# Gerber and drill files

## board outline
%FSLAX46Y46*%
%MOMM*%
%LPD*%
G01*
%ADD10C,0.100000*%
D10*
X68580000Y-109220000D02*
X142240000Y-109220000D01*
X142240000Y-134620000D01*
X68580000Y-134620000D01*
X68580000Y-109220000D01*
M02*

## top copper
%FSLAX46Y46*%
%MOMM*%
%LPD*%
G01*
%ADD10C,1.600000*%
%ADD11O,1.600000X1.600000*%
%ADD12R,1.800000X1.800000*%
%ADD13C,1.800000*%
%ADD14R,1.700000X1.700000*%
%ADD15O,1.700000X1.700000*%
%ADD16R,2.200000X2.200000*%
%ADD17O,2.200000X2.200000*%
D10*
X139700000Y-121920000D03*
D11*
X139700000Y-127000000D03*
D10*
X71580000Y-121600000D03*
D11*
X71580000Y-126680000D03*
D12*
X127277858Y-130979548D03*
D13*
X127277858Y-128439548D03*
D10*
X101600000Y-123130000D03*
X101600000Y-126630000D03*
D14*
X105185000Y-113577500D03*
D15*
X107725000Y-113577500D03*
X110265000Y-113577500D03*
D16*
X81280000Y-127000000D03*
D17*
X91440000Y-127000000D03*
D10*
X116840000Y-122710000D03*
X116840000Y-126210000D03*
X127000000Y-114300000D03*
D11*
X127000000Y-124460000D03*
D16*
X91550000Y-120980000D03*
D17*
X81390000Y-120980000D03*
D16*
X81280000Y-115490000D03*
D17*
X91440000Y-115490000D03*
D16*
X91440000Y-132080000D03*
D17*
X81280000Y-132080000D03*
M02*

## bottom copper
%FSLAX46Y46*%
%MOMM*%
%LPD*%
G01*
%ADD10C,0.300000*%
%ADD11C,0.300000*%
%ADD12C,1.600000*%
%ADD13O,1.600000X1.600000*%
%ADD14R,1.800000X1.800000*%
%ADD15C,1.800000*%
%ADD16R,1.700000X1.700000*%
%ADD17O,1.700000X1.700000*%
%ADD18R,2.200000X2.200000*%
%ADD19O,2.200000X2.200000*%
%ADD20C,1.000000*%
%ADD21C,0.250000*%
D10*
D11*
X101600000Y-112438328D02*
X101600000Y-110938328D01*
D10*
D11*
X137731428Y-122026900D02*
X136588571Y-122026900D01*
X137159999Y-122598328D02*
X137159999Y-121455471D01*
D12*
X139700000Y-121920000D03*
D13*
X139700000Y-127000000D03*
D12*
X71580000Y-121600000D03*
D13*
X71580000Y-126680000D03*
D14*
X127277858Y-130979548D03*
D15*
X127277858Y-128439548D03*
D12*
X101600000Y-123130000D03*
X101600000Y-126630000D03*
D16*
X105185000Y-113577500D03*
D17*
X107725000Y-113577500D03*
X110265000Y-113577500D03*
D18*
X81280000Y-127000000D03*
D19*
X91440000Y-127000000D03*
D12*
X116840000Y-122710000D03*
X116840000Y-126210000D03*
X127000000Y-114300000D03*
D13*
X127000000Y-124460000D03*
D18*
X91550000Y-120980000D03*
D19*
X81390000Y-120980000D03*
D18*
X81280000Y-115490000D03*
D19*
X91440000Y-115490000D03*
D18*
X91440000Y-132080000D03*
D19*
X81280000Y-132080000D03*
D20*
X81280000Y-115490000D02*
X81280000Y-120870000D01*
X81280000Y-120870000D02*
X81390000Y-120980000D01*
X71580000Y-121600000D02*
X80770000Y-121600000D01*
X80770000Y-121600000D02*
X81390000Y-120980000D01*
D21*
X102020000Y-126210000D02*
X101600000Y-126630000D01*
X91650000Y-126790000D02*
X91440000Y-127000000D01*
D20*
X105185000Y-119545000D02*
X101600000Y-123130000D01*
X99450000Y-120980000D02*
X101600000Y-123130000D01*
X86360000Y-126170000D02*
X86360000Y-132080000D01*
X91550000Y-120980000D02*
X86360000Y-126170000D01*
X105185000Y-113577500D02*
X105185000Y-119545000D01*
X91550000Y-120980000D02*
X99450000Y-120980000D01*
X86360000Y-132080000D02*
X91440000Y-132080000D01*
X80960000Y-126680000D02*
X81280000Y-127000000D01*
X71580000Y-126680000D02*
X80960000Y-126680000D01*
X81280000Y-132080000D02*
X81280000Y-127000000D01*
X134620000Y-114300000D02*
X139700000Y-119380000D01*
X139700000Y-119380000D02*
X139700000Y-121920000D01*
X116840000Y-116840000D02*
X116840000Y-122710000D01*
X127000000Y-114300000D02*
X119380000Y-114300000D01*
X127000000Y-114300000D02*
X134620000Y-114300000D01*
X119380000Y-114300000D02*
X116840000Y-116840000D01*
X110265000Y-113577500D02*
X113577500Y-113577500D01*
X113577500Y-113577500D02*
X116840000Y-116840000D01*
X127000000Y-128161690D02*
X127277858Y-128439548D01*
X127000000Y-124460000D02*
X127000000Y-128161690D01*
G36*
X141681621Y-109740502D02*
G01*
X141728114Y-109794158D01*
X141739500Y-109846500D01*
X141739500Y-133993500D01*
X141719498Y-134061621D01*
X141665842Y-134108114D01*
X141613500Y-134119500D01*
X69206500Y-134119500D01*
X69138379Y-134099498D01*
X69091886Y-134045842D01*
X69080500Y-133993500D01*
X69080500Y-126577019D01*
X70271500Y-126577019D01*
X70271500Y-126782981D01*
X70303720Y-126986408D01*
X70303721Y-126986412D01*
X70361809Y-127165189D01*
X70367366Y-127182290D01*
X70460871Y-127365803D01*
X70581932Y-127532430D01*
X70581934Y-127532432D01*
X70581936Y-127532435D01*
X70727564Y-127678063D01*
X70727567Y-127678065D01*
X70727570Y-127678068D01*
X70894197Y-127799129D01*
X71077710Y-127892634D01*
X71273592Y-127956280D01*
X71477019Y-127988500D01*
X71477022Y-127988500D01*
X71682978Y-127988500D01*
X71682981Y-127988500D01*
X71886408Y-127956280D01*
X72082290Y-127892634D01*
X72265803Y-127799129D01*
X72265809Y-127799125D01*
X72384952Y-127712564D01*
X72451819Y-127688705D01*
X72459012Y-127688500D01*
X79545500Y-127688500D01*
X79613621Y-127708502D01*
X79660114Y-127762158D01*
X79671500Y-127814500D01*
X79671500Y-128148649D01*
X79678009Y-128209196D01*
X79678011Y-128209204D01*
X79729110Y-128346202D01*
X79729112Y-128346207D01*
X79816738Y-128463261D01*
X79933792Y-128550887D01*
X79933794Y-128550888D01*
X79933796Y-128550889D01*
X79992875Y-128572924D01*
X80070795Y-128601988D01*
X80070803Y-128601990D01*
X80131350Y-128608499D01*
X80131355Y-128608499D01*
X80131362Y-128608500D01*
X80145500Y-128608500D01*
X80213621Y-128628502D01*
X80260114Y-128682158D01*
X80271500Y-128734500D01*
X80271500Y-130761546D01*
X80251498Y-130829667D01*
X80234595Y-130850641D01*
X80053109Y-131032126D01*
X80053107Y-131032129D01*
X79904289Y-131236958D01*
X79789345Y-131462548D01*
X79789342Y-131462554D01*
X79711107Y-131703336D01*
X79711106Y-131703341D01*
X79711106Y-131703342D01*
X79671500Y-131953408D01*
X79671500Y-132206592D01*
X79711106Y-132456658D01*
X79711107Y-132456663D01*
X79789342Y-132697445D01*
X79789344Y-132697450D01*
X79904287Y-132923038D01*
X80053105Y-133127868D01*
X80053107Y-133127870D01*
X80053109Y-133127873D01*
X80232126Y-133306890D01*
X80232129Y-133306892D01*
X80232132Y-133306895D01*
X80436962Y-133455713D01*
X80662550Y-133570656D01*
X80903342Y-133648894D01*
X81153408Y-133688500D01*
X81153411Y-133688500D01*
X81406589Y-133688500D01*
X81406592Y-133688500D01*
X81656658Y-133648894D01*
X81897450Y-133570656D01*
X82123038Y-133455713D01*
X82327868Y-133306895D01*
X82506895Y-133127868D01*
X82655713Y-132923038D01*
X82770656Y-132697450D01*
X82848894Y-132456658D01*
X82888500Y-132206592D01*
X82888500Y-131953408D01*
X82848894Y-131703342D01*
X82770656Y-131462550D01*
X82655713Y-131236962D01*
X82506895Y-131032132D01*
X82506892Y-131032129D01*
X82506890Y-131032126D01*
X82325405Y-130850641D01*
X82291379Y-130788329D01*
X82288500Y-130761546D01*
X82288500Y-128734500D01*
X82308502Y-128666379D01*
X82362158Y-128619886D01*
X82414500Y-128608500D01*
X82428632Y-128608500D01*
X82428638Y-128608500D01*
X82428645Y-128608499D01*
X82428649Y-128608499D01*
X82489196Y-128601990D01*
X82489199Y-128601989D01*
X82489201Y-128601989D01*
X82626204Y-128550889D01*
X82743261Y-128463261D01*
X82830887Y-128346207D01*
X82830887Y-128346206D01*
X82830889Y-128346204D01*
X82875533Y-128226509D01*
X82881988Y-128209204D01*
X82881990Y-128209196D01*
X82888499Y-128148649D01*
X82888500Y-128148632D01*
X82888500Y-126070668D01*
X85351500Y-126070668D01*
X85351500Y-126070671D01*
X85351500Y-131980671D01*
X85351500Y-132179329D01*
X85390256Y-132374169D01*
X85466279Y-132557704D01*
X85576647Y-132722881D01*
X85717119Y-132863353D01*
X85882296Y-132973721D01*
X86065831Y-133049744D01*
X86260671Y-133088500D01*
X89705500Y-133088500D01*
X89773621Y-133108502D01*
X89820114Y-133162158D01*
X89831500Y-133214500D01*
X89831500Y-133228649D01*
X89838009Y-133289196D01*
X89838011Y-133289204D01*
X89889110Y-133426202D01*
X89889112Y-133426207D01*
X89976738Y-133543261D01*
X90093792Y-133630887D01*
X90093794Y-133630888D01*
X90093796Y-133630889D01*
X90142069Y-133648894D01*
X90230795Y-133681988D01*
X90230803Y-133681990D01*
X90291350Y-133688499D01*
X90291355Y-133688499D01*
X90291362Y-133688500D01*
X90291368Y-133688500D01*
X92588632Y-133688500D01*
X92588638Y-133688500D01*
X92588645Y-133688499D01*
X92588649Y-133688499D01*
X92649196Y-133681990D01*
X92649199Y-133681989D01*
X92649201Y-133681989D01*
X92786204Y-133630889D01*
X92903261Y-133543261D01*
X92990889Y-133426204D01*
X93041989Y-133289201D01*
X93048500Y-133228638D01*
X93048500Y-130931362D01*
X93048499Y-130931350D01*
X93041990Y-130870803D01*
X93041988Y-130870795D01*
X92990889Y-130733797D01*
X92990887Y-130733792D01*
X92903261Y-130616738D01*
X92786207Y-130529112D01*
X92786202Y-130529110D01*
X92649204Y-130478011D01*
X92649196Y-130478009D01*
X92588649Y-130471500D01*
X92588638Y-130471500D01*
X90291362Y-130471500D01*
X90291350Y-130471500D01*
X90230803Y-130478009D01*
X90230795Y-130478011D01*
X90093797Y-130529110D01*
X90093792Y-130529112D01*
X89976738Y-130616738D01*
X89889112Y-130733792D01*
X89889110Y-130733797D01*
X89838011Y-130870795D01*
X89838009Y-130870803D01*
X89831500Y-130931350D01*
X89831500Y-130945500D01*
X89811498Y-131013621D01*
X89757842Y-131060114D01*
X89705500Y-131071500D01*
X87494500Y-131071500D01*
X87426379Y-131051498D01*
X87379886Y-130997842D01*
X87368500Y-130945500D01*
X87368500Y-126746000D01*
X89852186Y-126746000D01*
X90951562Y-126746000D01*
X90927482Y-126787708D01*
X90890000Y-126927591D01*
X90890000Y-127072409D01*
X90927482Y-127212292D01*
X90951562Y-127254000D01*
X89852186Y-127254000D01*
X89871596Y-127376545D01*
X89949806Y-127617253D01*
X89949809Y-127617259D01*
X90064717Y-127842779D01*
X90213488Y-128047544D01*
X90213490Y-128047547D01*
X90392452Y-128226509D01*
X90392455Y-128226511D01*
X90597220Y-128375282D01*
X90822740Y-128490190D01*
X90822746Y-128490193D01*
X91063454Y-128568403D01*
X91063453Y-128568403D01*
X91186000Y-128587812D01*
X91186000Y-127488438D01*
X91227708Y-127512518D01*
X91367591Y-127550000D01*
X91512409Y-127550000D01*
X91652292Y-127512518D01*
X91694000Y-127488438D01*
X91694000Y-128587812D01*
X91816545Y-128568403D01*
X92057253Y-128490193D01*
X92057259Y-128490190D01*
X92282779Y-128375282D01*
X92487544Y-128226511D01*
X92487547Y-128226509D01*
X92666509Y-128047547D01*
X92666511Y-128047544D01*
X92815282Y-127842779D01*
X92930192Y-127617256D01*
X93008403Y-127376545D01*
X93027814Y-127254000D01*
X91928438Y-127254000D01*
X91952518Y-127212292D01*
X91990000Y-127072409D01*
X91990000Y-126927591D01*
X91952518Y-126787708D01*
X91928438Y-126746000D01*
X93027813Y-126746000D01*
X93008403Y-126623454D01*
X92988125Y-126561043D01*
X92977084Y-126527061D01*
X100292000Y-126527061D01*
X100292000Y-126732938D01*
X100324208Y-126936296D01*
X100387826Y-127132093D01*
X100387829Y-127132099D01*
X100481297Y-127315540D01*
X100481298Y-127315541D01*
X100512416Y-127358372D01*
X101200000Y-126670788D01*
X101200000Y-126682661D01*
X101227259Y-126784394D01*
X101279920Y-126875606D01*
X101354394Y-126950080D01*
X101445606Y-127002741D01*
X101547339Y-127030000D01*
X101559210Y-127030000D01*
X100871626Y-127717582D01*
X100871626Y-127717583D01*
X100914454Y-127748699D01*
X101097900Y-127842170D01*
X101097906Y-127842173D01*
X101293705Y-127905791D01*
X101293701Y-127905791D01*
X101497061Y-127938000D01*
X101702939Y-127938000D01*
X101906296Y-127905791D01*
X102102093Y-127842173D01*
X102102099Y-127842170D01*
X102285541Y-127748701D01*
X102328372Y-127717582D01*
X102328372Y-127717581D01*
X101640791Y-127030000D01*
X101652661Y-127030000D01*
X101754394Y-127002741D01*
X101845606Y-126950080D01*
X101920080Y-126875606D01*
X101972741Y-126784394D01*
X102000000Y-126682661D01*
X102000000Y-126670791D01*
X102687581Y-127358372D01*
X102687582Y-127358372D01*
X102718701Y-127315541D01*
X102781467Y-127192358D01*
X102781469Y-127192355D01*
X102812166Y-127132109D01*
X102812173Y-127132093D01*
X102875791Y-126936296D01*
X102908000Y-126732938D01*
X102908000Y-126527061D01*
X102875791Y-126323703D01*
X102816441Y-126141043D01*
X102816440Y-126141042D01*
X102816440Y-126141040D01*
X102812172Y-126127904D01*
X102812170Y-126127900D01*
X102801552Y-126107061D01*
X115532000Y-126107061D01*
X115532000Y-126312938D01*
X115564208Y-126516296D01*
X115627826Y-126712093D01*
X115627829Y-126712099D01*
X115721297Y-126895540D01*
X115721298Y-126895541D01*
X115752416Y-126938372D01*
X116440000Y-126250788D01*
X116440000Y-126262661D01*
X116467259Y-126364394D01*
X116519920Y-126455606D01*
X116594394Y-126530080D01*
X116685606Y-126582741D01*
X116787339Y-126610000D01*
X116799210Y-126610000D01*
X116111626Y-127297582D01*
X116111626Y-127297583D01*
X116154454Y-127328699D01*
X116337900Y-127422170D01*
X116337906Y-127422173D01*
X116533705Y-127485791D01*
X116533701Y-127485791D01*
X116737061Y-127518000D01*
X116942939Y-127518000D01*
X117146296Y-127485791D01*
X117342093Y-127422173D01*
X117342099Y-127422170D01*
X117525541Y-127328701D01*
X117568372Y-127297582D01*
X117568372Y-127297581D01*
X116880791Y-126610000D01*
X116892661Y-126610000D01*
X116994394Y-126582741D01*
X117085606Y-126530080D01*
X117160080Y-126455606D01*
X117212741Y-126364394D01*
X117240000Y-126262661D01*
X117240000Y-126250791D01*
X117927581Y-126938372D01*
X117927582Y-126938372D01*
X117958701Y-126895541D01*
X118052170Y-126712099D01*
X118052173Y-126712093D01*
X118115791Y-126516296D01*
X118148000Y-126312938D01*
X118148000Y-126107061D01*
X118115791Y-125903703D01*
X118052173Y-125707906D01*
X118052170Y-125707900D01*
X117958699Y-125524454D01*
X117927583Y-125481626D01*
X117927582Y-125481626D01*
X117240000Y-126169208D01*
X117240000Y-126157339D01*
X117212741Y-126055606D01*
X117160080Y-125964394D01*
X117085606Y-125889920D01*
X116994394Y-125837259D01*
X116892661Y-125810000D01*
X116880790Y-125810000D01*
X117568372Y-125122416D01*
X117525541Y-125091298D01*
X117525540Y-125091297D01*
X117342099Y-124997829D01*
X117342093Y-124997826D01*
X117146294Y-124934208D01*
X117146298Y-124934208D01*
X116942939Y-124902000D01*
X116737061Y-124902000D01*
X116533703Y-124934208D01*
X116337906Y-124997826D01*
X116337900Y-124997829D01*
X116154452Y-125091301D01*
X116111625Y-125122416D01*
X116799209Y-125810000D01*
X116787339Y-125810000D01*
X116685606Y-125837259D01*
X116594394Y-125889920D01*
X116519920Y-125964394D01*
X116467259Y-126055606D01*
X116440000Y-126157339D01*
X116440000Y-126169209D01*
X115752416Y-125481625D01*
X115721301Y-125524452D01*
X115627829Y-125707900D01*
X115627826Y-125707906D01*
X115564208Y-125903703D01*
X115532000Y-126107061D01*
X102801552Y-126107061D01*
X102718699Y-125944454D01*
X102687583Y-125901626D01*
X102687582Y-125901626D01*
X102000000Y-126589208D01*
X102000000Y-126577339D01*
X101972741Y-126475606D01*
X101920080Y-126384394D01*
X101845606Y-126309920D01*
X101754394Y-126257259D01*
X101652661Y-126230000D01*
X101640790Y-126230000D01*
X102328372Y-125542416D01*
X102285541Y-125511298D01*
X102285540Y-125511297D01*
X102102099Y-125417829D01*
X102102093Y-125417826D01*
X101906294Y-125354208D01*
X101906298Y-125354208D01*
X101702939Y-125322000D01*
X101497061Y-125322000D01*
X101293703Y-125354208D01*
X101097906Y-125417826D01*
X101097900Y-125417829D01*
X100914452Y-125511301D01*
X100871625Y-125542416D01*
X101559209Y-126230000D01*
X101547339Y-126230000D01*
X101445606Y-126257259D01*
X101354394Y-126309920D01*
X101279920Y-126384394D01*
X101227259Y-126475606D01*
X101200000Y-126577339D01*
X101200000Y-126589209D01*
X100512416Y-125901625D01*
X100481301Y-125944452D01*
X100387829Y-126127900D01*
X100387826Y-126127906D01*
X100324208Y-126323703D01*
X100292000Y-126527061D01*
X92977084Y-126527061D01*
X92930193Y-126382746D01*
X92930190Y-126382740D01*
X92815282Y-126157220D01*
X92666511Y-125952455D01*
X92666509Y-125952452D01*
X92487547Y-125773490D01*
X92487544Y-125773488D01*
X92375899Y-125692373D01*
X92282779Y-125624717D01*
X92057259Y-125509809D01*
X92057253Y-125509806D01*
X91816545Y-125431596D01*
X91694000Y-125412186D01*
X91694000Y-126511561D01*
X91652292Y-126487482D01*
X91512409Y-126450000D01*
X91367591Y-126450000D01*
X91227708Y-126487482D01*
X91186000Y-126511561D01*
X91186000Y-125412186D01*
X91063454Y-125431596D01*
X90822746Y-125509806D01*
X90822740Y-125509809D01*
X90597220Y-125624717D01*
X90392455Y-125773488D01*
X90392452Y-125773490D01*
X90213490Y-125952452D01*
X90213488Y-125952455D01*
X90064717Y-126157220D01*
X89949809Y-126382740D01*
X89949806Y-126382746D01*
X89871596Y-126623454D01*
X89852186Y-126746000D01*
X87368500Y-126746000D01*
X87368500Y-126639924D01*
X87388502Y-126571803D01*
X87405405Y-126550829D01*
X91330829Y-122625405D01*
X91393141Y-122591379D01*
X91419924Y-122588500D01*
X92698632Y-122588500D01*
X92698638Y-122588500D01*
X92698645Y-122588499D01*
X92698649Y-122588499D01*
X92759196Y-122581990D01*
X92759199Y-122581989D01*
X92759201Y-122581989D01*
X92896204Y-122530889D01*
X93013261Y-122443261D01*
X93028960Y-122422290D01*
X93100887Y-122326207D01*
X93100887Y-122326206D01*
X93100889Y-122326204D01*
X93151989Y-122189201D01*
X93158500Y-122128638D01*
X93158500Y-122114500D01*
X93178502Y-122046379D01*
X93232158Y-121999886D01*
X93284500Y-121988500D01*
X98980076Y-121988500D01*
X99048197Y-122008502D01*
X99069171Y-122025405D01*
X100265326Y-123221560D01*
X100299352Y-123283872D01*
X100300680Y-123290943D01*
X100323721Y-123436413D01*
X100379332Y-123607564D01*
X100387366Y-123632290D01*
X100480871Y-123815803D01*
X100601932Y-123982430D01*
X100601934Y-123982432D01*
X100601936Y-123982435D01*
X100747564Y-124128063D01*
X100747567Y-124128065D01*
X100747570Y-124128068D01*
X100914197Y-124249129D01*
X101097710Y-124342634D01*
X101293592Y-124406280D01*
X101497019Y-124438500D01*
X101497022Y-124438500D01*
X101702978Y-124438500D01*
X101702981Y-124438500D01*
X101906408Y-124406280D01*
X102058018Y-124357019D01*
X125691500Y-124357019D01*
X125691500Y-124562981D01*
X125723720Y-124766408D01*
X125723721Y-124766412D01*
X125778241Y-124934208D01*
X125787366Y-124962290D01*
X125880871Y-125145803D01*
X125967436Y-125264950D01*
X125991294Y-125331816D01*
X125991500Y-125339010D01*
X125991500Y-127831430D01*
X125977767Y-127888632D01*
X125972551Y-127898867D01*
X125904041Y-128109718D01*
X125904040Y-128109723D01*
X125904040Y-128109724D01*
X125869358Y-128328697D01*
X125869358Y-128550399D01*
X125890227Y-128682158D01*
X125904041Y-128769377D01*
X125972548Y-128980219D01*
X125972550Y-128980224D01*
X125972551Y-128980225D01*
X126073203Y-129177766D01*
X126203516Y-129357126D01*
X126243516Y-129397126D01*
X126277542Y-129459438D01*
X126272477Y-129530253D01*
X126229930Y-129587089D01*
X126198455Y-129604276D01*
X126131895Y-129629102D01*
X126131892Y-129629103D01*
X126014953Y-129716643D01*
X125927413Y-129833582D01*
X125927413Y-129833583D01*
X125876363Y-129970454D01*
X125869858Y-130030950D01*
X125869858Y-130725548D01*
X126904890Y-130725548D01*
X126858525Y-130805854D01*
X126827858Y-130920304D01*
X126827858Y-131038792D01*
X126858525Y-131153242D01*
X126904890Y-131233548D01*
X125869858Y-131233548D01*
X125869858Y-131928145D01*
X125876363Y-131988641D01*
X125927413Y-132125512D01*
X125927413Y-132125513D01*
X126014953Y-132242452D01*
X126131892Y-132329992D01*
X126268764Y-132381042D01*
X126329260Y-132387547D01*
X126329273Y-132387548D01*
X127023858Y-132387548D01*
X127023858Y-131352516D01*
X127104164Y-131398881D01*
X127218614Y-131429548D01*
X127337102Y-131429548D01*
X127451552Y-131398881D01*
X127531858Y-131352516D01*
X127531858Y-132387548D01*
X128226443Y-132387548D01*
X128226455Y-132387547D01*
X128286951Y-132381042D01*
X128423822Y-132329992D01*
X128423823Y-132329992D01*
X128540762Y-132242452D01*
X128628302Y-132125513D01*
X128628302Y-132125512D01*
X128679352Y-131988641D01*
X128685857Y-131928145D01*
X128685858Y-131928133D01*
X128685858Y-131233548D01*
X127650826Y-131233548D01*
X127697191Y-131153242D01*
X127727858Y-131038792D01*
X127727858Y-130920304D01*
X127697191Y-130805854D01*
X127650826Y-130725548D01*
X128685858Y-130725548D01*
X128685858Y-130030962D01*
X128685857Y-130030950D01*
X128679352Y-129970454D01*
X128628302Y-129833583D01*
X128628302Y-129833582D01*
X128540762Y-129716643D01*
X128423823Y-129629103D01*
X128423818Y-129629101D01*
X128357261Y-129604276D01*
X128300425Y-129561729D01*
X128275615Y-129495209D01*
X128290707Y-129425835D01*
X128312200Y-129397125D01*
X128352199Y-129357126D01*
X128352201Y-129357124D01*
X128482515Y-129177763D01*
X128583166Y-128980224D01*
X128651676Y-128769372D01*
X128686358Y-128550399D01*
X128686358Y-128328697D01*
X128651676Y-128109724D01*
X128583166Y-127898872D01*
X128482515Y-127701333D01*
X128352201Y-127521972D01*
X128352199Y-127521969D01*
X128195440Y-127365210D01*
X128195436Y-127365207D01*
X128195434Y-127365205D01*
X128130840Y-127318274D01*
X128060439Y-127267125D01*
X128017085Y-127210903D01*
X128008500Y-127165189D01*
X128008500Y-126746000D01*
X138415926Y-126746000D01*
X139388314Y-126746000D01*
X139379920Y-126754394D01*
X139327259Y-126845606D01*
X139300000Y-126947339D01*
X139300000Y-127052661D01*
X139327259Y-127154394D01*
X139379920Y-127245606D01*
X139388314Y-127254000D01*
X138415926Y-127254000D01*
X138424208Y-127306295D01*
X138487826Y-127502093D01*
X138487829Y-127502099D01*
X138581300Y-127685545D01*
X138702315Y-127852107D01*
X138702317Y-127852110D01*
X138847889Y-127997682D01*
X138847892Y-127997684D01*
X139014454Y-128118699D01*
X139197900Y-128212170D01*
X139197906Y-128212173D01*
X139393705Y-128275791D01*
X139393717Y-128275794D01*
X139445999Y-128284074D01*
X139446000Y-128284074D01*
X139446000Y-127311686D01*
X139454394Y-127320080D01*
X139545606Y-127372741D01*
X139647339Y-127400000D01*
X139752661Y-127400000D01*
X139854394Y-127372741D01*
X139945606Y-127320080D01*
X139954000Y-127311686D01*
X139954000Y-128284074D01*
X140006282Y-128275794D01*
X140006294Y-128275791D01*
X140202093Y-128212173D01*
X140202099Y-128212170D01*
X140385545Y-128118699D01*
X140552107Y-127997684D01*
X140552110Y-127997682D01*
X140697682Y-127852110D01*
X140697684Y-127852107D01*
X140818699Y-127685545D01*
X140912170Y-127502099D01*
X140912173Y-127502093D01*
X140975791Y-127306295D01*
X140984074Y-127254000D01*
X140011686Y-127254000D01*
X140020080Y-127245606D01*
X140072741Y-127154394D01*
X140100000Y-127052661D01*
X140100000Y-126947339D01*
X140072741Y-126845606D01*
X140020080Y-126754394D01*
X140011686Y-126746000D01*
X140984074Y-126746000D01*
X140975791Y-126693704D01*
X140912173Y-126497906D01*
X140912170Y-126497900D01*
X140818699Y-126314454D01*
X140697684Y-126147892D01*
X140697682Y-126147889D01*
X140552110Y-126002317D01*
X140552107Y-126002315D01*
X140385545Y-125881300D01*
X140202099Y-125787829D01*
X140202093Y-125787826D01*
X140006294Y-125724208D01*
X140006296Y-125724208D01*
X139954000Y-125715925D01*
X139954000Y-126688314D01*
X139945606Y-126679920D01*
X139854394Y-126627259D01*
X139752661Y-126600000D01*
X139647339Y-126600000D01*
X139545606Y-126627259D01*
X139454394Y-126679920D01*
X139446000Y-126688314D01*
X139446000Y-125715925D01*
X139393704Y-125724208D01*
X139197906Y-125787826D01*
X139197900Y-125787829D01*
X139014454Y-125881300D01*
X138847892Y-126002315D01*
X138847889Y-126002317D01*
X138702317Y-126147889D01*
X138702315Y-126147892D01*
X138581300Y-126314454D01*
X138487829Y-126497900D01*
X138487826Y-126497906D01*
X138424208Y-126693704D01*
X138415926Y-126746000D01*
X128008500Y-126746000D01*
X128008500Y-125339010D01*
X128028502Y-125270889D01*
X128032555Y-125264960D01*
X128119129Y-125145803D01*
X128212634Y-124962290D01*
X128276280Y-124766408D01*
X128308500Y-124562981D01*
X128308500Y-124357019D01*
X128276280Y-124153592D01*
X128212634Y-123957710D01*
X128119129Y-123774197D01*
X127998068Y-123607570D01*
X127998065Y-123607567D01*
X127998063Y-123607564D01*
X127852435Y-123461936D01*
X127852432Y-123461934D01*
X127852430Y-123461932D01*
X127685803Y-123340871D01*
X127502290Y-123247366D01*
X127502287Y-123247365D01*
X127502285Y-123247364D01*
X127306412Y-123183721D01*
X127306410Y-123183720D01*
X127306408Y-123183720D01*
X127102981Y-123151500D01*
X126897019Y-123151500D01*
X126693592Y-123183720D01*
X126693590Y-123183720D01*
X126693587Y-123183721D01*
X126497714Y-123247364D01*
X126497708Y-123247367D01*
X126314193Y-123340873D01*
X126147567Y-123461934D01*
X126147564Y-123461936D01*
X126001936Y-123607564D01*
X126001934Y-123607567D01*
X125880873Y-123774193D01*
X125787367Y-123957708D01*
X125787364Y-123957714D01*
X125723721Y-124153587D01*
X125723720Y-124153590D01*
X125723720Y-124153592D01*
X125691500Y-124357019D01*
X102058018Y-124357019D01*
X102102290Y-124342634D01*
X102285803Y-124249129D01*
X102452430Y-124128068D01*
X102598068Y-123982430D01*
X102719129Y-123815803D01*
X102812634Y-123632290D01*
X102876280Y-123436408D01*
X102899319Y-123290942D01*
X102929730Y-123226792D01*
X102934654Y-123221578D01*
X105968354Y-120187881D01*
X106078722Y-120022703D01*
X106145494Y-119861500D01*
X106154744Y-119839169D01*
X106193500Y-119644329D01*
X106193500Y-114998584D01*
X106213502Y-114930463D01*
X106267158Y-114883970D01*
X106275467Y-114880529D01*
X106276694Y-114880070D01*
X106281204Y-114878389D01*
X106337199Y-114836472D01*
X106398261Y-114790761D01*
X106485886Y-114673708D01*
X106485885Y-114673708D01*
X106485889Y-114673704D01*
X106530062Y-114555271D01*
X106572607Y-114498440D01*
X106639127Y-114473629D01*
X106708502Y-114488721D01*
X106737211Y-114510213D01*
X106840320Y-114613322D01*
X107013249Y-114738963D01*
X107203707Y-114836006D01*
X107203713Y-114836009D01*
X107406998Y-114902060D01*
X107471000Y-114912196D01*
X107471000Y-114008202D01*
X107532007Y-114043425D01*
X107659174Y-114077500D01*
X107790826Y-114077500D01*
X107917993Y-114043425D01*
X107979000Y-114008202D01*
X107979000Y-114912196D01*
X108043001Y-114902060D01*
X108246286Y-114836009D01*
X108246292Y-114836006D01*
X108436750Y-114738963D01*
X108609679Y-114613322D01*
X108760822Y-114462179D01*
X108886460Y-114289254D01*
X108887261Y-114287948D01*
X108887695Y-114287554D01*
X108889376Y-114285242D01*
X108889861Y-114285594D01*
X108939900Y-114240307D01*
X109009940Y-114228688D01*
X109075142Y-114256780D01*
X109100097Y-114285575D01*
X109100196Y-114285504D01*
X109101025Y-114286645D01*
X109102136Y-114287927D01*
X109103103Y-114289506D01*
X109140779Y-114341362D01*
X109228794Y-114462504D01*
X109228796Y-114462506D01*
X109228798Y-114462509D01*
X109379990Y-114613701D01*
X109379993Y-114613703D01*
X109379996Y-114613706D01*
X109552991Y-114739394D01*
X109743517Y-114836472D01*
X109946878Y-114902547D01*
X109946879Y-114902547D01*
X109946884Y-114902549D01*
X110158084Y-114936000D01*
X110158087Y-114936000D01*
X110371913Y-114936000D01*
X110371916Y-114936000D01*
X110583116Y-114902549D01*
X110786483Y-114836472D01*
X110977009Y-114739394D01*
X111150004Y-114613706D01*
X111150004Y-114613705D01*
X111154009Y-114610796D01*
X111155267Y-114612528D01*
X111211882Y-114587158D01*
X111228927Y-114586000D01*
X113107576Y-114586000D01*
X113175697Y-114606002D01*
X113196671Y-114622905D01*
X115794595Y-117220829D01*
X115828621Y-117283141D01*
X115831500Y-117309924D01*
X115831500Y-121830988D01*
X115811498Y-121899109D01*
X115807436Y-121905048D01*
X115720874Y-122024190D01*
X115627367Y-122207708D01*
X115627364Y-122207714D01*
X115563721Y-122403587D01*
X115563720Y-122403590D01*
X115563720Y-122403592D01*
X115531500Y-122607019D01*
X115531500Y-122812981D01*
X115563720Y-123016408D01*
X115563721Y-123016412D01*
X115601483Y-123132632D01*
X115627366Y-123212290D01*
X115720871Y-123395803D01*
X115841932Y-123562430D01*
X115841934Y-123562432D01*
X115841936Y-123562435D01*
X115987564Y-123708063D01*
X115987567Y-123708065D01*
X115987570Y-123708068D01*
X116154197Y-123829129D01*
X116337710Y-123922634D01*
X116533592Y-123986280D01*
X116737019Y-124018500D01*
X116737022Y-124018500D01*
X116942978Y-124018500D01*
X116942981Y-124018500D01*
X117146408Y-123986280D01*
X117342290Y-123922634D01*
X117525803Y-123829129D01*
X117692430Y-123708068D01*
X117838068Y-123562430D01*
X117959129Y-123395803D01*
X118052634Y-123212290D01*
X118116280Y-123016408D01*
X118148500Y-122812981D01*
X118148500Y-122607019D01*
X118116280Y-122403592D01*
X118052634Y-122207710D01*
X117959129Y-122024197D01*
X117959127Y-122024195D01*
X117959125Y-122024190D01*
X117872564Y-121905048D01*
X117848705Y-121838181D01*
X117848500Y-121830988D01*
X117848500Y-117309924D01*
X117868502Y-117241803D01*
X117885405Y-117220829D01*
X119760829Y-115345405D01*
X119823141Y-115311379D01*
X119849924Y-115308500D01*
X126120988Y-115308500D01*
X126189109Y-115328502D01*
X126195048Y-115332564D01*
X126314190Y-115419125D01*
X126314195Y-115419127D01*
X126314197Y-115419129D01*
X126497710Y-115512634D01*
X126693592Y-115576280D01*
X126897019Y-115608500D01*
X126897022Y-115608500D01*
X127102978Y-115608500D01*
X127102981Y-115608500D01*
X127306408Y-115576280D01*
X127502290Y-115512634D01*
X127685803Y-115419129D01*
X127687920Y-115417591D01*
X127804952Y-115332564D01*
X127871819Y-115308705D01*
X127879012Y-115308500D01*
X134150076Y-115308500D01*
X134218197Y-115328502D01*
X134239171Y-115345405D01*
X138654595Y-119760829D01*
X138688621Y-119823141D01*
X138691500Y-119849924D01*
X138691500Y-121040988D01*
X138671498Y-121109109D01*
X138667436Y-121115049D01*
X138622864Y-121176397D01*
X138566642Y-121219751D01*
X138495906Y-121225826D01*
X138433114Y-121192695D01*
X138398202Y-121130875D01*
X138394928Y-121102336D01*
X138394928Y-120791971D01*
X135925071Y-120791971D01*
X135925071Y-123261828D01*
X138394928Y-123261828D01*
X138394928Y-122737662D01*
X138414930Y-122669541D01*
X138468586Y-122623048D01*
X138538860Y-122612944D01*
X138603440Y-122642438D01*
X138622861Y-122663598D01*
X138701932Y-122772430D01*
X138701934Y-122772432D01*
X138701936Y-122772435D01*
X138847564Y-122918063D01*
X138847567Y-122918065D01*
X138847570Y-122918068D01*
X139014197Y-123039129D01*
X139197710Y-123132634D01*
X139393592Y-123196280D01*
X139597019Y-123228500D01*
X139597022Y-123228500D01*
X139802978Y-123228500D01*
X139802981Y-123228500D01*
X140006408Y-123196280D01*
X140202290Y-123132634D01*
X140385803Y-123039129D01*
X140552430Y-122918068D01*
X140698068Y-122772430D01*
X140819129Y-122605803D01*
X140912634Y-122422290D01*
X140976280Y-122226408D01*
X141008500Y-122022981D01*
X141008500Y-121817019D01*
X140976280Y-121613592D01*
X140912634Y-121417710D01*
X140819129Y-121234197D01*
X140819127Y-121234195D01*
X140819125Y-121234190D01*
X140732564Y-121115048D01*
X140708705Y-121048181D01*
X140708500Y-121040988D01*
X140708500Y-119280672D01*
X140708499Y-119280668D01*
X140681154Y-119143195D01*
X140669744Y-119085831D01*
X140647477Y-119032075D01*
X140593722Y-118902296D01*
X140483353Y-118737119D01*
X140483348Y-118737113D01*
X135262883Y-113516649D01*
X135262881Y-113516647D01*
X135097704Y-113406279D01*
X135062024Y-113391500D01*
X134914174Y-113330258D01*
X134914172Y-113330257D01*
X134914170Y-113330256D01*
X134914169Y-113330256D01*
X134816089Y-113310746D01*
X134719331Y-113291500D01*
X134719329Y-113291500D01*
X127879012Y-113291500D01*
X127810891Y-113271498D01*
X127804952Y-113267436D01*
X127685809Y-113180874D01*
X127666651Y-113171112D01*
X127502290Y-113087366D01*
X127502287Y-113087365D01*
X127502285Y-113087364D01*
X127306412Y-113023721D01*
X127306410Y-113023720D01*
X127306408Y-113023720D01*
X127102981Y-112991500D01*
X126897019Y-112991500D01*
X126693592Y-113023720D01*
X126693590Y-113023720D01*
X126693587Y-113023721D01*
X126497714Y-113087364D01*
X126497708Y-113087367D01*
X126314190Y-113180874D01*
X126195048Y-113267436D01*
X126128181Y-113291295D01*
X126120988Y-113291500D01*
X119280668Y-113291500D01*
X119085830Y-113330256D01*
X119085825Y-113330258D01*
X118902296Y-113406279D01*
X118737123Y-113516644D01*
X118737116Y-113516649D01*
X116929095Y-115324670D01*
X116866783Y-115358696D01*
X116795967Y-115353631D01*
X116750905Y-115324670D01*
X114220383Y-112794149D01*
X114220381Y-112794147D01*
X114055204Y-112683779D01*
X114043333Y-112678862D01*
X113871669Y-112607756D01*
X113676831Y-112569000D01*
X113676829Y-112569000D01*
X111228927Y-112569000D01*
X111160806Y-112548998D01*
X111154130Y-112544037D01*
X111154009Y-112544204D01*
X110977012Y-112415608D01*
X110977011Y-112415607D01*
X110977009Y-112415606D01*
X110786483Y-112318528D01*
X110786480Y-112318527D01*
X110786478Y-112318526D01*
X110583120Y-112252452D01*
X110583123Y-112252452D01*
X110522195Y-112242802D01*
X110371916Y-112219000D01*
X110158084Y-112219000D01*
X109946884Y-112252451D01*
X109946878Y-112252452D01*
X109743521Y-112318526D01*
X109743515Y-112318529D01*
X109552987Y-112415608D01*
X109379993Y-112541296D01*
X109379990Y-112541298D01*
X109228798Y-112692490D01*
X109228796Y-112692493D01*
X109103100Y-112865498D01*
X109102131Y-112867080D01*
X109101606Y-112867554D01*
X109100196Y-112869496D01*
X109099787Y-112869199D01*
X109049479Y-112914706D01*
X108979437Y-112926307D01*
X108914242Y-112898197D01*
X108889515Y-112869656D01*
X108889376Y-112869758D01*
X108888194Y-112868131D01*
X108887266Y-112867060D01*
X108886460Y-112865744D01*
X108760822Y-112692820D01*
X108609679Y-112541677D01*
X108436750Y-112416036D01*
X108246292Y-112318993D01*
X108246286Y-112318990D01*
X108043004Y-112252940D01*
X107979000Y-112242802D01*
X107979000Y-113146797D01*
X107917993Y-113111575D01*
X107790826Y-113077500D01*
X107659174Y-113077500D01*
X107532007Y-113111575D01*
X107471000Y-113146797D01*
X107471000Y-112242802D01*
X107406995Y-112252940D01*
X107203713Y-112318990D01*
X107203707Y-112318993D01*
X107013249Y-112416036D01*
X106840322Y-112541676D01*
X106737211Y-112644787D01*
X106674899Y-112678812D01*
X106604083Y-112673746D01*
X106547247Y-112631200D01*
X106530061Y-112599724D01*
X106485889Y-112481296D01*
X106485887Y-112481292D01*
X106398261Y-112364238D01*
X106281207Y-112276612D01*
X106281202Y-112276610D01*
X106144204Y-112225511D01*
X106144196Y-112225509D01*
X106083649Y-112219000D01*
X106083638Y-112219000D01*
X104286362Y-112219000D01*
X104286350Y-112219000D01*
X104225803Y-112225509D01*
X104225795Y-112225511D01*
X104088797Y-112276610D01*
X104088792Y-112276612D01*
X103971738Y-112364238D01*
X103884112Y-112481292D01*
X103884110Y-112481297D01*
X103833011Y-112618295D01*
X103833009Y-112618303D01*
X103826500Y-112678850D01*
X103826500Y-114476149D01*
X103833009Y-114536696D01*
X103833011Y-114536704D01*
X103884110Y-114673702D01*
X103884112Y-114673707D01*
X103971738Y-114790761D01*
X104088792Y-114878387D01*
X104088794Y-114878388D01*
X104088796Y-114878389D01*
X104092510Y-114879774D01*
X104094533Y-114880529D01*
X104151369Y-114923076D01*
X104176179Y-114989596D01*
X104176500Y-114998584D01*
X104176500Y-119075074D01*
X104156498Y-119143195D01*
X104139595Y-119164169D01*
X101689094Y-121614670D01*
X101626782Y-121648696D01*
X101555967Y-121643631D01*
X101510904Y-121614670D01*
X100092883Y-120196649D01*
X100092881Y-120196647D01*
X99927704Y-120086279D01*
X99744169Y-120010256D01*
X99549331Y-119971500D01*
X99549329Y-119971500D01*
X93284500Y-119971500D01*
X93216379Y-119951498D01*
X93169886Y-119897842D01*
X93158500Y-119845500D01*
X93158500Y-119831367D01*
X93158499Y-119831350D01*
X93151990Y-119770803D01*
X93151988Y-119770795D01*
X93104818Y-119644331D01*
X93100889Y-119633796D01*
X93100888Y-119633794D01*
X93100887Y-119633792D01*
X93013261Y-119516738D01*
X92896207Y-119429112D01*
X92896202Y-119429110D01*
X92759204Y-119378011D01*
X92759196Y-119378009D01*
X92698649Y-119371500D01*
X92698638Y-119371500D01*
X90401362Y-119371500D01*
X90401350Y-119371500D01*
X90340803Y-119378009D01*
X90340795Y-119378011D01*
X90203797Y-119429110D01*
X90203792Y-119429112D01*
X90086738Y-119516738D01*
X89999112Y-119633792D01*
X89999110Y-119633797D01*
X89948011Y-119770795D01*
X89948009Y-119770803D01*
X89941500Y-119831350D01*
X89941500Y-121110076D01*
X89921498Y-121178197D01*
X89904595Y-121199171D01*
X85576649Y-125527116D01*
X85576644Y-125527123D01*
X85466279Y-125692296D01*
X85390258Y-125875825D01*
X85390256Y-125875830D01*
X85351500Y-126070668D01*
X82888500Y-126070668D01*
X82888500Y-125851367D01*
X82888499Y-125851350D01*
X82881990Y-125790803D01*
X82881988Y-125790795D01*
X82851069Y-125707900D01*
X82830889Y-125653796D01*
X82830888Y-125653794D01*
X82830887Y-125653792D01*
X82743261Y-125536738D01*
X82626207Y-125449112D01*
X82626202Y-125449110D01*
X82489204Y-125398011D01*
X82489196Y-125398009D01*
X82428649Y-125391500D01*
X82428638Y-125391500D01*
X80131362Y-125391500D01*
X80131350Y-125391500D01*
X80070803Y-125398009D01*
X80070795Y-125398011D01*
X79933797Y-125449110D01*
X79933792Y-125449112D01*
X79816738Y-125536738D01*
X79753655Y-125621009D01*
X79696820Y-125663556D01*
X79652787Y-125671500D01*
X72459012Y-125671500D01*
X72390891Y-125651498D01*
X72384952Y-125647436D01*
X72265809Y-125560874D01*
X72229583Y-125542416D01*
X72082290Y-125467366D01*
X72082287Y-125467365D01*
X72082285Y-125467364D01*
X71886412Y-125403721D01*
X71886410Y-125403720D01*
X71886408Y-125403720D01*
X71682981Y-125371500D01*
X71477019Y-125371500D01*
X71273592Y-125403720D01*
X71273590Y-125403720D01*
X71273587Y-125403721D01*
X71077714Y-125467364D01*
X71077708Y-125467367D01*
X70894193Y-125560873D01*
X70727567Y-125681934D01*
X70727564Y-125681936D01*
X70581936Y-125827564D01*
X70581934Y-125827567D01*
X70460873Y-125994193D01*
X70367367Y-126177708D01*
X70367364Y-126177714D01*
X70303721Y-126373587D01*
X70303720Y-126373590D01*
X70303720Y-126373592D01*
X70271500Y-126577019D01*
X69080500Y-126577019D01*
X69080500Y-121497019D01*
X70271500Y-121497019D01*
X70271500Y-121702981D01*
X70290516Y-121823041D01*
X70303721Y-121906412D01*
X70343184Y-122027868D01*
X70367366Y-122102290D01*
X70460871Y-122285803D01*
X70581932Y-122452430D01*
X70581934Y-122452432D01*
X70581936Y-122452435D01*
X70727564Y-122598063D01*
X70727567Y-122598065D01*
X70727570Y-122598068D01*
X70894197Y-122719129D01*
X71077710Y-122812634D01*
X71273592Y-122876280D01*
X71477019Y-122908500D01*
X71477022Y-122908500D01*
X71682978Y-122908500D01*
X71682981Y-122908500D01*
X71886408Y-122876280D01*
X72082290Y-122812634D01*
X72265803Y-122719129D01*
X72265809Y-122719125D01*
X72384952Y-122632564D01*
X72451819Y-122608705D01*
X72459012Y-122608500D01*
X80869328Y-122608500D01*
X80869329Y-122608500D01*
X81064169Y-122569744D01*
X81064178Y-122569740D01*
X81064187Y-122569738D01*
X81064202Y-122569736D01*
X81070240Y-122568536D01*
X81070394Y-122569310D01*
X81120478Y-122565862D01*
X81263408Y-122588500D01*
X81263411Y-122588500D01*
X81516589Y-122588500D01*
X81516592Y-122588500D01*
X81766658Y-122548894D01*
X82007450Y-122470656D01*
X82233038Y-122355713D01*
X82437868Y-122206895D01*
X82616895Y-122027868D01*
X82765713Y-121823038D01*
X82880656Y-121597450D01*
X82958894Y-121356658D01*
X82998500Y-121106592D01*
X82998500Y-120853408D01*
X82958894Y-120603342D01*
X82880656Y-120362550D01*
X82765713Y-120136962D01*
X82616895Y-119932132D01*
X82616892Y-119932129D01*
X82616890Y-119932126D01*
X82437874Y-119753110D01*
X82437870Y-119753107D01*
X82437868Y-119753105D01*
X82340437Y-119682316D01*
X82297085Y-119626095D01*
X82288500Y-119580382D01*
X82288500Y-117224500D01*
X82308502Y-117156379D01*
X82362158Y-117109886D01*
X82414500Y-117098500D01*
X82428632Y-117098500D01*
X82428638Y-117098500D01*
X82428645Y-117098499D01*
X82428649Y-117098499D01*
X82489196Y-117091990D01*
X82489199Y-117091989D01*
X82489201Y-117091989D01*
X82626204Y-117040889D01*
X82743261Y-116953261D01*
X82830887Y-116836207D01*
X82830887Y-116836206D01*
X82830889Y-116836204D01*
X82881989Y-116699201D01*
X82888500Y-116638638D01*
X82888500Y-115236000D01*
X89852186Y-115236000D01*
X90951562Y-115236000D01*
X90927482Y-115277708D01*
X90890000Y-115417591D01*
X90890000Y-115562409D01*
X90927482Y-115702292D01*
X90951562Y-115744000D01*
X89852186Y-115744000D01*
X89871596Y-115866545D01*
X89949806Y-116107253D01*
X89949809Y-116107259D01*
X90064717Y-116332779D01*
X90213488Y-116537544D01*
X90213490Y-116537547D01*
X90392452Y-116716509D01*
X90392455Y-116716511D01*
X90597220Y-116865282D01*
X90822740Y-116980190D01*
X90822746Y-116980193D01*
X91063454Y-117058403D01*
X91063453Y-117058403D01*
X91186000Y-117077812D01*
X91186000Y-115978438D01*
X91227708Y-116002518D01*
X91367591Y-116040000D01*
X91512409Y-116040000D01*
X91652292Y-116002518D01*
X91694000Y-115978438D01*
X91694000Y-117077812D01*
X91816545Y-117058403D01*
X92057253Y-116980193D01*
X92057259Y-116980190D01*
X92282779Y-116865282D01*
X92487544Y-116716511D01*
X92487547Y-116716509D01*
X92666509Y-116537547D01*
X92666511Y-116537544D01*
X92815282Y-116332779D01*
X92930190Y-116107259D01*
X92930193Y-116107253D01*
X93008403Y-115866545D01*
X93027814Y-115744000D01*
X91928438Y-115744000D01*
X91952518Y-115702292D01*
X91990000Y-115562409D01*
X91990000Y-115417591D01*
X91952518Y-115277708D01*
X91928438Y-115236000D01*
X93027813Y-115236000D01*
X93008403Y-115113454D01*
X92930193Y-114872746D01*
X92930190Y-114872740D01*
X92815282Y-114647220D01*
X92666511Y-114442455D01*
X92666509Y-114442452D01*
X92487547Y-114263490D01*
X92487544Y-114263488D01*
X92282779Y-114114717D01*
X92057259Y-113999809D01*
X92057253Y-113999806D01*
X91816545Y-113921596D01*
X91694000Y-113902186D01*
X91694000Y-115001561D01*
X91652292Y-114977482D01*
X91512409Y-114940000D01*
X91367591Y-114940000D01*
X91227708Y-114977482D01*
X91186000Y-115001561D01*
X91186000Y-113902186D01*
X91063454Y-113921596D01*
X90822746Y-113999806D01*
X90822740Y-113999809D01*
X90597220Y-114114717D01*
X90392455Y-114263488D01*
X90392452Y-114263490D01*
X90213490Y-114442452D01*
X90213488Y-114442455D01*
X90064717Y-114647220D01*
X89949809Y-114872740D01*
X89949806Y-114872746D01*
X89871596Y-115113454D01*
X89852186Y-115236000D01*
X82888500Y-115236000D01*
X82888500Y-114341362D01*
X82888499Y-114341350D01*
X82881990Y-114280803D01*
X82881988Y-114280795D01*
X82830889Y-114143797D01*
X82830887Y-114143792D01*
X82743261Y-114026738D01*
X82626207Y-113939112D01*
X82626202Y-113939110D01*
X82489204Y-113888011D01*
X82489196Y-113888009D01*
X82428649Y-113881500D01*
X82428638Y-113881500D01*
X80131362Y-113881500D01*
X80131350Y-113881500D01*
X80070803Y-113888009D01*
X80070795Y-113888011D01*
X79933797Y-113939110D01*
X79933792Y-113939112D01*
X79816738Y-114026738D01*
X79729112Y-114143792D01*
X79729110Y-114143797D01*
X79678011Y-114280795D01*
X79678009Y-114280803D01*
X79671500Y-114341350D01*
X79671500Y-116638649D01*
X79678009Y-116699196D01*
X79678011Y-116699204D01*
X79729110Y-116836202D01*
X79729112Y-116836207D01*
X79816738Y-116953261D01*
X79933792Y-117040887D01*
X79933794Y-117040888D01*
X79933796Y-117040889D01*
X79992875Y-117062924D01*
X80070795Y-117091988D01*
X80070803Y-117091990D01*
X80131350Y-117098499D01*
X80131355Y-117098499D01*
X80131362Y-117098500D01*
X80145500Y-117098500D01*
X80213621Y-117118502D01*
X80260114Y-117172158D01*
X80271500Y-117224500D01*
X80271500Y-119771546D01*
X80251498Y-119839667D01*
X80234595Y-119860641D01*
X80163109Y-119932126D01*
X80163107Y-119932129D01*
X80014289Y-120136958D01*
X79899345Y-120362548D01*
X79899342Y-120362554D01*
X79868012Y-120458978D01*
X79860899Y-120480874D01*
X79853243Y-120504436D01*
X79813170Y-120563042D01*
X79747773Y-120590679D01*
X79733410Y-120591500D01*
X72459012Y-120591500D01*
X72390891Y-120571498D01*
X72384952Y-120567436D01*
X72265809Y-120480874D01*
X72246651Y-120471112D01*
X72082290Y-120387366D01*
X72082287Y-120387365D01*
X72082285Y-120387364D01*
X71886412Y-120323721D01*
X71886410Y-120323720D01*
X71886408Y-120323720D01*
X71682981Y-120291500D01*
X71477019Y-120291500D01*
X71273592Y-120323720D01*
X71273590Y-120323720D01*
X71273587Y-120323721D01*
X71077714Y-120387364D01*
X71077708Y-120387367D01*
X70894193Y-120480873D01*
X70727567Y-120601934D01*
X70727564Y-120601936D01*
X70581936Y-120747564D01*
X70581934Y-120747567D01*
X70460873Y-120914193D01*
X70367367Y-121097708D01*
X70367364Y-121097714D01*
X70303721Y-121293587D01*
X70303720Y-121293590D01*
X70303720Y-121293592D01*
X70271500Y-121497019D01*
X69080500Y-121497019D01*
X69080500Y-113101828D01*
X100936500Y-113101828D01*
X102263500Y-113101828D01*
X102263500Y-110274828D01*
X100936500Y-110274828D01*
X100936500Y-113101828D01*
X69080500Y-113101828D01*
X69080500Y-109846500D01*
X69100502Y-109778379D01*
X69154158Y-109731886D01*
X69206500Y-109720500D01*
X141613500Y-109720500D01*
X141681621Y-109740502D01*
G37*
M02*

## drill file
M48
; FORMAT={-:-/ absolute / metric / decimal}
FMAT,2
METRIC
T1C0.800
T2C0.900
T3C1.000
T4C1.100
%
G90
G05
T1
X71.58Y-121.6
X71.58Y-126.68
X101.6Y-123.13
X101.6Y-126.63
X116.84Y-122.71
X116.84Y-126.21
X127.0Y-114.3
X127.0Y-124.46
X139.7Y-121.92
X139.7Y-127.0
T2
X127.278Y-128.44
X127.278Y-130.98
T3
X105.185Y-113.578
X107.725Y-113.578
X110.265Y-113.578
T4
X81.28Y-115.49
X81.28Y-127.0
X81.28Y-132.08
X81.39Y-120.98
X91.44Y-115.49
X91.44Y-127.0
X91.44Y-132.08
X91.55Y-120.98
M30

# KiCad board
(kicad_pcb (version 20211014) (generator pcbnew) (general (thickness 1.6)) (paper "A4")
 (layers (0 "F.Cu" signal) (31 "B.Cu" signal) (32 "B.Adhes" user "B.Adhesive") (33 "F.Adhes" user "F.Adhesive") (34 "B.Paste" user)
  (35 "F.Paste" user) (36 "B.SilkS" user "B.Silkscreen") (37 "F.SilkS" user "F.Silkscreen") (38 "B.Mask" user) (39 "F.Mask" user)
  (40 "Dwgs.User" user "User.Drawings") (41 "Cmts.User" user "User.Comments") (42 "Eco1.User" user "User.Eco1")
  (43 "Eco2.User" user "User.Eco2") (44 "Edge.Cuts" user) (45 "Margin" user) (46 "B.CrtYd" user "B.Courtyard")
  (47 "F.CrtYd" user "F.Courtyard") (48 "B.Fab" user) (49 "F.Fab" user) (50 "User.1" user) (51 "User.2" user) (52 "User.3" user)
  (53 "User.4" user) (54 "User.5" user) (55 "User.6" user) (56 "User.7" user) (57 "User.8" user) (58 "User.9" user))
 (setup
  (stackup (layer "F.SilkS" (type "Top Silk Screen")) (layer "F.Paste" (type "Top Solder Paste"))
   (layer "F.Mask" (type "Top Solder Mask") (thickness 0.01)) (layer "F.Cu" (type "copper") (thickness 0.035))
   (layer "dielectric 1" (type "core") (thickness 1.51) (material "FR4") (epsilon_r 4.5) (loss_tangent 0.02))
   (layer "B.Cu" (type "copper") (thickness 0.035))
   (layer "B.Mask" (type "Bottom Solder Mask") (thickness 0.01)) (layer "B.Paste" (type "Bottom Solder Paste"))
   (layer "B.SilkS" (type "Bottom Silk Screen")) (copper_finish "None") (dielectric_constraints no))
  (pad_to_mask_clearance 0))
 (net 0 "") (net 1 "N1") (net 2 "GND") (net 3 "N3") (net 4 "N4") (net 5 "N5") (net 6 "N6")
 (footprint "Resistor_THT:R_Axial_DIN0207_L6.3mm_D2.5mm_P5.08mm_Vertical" (layer "F.Cu") (at 139.7 121.92 -90)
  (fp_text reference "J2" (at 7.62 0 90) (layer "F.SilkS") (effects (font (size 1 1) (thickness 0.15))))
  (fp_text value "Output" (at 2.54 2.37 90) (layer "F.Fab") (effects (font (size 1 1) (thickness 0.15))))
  (pad "1" thru_hole circle (at 0 0 270) (size 1.6 1.6) (drill 0.8) (layers *.Cu *.Mask) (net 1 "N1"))
  (pad "2" thru_hole oval (at 5.08 0 270) (size 1.6 1.6) (drill 0.8) (layers *.Cu *.Mask) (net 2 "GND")))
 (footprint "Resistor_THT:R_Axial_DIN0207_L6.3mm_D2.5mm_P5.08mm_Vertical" (layer "F.Cu") (at 71.58 121.6 -90)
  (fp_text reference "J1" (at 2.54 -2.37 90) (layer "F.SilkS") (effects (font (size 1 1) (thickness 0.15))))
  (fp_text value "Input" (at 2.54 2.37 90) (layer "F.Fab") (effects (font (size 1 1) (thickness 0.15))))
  (pad "1" thru_hole circle (at 0 0 270) (size 1.6 1.6) (drill 0.8) (layers *.Cu *.Mask) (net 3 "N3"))
  (pad "2" thru_hole oval (at 5.08 0 270) (size 1.6 1.6) (drill 0.8) (layers *.Cu *.Mask) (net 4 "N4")))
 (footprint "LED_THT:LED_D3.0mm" (layer "F.Cu") (at 127.277858 130.979548 90)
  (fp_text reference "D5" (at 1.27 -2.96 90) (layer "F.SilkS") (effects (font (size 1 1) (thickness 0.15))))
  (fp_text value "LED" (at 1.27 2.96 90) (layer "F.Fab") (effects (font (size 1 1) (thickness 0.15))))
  (pad "1" thru_hole rect (at 0 0 90) (size 1.8 1.8) (drill 0.9) (layers *.Cu *.Mask) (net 2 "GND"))
  (pad "2" thru_hole circle (at 2.54 0 90) (size 1.8 1.8) (drill 0.9) (layers *.Cu *.Mask) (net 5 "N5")))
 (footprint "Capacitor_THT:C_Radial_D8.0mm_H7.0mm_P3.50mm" (layer "F.Cu") (at 101.6 123.13 -90)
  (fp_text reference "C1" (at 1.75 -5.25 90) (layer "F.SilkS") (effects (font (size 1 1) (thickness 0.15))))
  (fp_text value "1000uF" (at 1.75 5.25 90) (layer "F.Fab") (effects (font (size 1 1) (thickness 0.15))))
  (pad "1" thru_hole circle (at 0 0 270) (size 1.6 1.6) (drill 0.8) (layers *.Cu *.Mask) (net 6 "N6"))
  (pad "2" thru_hole circle (at 3.5 0 270) (size 1.6 1.6) (drill 0.8) (layers *.Cu *.Mask) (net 2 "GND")))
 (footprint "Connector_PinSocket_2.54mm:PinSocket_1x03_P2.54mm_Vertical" (layer "F.Cu") (at 105.185 113.5775 90)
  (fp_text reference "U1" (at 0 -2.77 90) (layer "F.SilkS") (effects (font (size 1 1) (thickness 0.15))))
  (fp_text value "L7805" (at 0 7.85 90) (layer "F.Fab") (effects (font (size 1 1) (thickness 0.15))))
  (pad "1" thru_hole rect (at 0 0 90) (size 1.7 1.7) (drill 1) (layers *.Cu *.Mask) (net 6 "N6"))
  (pad "2" thru_hole oval (at 0 2.54 90) (size 1.7 1.7) (drill 1) (layers *.Cu *.Mask) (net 2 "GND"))
  (pad "3" thru_hole oval (at 0 5.08 90) (size 1.7 1.7) (drill 1) (layers *.Cu *.Mask) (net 1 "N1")))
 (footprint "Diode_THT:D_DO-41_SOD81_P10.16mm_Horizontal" (layer "F.Cu") (at 81.28 127)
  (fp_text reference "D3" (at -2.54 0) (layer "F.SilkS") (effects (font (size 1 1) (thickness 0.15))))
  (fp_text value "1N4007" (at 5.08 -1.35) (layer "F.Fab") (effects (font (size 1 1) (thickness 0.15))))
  (pad "1" thru_hole rect (at 0 0) (size 2.2 2.2) (drill 1.1) (layers *.Cu *.Mask) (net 4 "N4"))
  (pad "2" thru_hole oval (at 10.16 0) (size 2.2 2.2) (drill 1.1) (layers *.Cu *.Mask) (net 2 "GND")))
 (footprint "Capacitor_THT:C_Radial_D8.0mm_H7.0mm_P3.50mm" (layer "F.Cu") (at 116.84 122.71 -90)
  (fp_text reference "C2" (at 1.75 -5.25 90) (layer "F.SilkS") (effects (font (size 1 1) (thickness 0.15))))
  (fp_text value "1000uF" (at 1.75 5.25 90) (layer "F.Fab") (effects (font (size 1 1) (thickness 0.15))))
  (pad "1" thru_hole circle (at 0 0 270) (size 1.6 1.6) (drill 0.8) (layers *.Cu *.Mask) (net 1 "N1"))
  (pad "2" thru_hole circle (at 3.5 0 270) (size 1.6 1.6) (drill 0.8) (layers *.Cu *.Mask) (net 2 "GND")))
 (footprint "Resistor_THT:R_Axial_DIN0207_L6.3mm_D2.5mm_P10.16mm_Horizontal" (layer "F.Cu") (at 127 114.3 -90)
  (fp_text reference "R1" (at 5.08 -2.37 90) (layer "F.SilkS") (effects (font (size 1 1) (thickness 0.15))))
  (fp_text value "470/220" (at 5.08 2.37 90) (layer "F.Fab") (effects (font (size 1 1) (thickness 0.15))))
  (pad "1" thru_hole circle (at 0 0 270) (size 1.6 1.6) (drill 0.8) (layers *.Cu *.Mask) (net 1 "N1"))
  (pad "2" thru_hole oval (at 10.16 0 270) (size 1.6 1.6) (drill 0.8) (layers *.Cu *.Mask) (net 5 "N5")))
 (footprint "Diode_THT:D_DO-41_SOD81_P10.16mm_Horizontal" (layer "F.Cu") (at 91.55 120.98 180)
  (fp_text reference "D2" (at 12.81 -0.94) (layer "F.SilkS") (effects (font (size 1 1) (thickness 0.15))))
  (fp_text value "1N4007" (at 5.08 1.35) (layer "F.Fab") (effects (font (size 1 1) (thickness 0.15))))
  (pad "1" thru_hole rect (at 0 0 180) (size 2.2 2.2) (drill 1.1) (layers *.Cu *.Mask) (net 6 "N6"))
  (pad "2" thru_hole oval (at 10.16 0 180) (size 2.2 2.2) (drill 1.1) (layers *.Cu *.Mask) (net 3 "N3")))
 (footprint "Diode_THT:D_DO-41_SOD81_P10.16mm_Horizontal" (layer "F.Cu") (at 81.28 115.49)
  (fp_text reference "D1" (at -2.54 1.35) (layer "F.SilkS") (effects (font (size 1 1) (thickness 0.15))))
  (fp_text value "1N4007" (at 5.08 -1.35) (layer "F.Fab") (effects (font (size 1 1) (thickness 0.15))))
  (pad "1" thru_hole rect (at 0 0) (size 2.2 2.2) (drill 1.1) (layers *.Cu *.Mask) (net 3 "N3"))
  (pad "2" thru_hole oval (at 10.16 0) (size 2.2 2.2) (drill 1.1) (layers *.Cu *.Mask) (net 2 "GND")))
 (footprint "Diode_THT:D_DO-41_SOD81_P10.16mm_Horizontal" (layer "F.Cu") (at 91.44 132.08 180)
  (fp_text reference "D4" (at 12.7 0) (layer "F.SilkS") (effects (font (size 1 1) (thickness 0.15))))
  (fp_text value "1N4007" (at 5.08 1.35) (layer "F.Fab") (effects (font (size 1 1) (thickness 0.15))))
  (pad "1" thru_hole rect (at 0 0 180) (size 2.2 2.2) (drill 1.1) (layers *.Cu *.Mask) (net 6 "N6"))
  (pad "2" thru_hole oval (at 10.16 0 180) (size 2.2 2.2) (drill 1.1) (layers *.Cu *.Mask) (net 4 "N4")))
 (gr_rect (start 68.58 109.22) (end 142.24 134.62) (layer "Edge.Cuts") (width 0.1) (fill none))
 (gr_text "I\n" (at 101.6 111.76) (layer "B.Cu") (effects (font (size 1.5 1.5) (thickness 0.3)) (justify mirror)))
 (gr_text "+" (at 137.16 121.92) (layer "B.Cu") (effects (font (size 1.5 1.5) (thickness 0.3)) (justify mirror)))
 (segment (start 81.28 115.49) (end 81.28 120.87) (width 1) (layer "B.Cu") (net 3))
 (segment (start 81.28 120.87) (end 81.39 120.98) (width 1) (layer "B.Cu") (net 3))
 (segment (start 71.58 121.6) (end 80.77 121.6) (width 1) (layer "B.Cu") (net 3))
 (segment (start 80.77 121.6) (end 81.39 120.98) (width 1) (layer "B.Cu") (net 3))
 (segment (start 102.02 126.21) (end 101.6 126.63) (width 0.25) (layer "B.Cu") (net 2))
 (segment (start 91.65 126.79) (end 91.44 127) (width 0.25) (layer "B.Cu") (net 2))
 (segment (start 105.185 119.545) (end 101.6 123.13) (width 1) (layer "B.Cu") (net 6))
 (segment (start 99.45 120.98) (end 101.6 123.13) (width 1) (layer "B.Cu") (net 6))
 (segment (start 86.36 126.17) (end 86.36 132.08) (width 1) (layer "B.Cu") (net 6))
 (segment (start 91.55 120.98) (end 86.36 126.17) (width 1) (layer "B.Cu") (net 6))
 (segment (start 105.185 113.5775) (end 105.185 119.545) (width 1) (layer "B.Cu") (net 6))
 (segment (start 91.55 120.98) (end 99.45 120.98) (width 1) (layer "B.Cu") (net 6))
 (segment (start 86.36 132.08) (end 91.44 132.08) (width 1) (layer "B.Cu") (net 6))
 (segment (start 80.96 126.68) (end 81.28 127) (width 1) (layer "B.Cu") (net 4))
 (segment (start 71.58 126.68) (end 80.96 126.68) (width 1) (layer "B.Cu") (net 4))
 (segment (start 81.28 132.08) (end 81.28 127) (width 1) (layer "B.Cu") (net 4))
 (segment (start 134.62 114.3) (end 139.7 119.38) (width 1) (layer "B.Cu") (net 1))
 (segment (start 139.7 119.38) (end 139.7 121.92) (width 1) (layer "B.Cu") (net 1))
 (segment (start 116.84 116.84) (end 116.84 122.71) (width 1) (layer "B.Cu") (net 1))
 (segment (start 127 114.3) (end 119.38 114.3) (width 1) (layer "B.Cu") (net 1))
 (segment (start 127 114.3) (end 134.62 114.3) (width 1) (layer "B.Cu") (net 1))
 (segment (start 119.38 114.3) (end 116.84 116.84) (width 1) (layer "B.Cu") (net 1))
 (segment (start 110.265 113.5775) (end 113.5775 113.5775) (width 1) (layer "B.Cu") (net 1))
 (segment (start 113.5775 113.5775) (end 116.84 116.84) (width 1) (layer "B.Cu") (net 1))
 (segment (start 127 128.16169) (end 127.277858 128.439548) (width 1) (layer "B.Cu") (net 5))
 (segment (start 127 124.46) (end 127 128.16169) (width 1) (layer "B.Cu") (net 5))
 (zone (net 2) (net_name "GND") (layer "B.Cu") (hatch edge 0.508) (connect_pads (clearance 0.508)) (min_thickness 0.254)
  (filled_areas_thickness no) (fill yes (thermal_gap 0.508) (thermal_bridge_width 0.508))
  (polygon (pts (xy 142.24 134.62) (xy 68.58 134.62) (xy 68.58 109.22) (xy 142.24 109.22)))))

